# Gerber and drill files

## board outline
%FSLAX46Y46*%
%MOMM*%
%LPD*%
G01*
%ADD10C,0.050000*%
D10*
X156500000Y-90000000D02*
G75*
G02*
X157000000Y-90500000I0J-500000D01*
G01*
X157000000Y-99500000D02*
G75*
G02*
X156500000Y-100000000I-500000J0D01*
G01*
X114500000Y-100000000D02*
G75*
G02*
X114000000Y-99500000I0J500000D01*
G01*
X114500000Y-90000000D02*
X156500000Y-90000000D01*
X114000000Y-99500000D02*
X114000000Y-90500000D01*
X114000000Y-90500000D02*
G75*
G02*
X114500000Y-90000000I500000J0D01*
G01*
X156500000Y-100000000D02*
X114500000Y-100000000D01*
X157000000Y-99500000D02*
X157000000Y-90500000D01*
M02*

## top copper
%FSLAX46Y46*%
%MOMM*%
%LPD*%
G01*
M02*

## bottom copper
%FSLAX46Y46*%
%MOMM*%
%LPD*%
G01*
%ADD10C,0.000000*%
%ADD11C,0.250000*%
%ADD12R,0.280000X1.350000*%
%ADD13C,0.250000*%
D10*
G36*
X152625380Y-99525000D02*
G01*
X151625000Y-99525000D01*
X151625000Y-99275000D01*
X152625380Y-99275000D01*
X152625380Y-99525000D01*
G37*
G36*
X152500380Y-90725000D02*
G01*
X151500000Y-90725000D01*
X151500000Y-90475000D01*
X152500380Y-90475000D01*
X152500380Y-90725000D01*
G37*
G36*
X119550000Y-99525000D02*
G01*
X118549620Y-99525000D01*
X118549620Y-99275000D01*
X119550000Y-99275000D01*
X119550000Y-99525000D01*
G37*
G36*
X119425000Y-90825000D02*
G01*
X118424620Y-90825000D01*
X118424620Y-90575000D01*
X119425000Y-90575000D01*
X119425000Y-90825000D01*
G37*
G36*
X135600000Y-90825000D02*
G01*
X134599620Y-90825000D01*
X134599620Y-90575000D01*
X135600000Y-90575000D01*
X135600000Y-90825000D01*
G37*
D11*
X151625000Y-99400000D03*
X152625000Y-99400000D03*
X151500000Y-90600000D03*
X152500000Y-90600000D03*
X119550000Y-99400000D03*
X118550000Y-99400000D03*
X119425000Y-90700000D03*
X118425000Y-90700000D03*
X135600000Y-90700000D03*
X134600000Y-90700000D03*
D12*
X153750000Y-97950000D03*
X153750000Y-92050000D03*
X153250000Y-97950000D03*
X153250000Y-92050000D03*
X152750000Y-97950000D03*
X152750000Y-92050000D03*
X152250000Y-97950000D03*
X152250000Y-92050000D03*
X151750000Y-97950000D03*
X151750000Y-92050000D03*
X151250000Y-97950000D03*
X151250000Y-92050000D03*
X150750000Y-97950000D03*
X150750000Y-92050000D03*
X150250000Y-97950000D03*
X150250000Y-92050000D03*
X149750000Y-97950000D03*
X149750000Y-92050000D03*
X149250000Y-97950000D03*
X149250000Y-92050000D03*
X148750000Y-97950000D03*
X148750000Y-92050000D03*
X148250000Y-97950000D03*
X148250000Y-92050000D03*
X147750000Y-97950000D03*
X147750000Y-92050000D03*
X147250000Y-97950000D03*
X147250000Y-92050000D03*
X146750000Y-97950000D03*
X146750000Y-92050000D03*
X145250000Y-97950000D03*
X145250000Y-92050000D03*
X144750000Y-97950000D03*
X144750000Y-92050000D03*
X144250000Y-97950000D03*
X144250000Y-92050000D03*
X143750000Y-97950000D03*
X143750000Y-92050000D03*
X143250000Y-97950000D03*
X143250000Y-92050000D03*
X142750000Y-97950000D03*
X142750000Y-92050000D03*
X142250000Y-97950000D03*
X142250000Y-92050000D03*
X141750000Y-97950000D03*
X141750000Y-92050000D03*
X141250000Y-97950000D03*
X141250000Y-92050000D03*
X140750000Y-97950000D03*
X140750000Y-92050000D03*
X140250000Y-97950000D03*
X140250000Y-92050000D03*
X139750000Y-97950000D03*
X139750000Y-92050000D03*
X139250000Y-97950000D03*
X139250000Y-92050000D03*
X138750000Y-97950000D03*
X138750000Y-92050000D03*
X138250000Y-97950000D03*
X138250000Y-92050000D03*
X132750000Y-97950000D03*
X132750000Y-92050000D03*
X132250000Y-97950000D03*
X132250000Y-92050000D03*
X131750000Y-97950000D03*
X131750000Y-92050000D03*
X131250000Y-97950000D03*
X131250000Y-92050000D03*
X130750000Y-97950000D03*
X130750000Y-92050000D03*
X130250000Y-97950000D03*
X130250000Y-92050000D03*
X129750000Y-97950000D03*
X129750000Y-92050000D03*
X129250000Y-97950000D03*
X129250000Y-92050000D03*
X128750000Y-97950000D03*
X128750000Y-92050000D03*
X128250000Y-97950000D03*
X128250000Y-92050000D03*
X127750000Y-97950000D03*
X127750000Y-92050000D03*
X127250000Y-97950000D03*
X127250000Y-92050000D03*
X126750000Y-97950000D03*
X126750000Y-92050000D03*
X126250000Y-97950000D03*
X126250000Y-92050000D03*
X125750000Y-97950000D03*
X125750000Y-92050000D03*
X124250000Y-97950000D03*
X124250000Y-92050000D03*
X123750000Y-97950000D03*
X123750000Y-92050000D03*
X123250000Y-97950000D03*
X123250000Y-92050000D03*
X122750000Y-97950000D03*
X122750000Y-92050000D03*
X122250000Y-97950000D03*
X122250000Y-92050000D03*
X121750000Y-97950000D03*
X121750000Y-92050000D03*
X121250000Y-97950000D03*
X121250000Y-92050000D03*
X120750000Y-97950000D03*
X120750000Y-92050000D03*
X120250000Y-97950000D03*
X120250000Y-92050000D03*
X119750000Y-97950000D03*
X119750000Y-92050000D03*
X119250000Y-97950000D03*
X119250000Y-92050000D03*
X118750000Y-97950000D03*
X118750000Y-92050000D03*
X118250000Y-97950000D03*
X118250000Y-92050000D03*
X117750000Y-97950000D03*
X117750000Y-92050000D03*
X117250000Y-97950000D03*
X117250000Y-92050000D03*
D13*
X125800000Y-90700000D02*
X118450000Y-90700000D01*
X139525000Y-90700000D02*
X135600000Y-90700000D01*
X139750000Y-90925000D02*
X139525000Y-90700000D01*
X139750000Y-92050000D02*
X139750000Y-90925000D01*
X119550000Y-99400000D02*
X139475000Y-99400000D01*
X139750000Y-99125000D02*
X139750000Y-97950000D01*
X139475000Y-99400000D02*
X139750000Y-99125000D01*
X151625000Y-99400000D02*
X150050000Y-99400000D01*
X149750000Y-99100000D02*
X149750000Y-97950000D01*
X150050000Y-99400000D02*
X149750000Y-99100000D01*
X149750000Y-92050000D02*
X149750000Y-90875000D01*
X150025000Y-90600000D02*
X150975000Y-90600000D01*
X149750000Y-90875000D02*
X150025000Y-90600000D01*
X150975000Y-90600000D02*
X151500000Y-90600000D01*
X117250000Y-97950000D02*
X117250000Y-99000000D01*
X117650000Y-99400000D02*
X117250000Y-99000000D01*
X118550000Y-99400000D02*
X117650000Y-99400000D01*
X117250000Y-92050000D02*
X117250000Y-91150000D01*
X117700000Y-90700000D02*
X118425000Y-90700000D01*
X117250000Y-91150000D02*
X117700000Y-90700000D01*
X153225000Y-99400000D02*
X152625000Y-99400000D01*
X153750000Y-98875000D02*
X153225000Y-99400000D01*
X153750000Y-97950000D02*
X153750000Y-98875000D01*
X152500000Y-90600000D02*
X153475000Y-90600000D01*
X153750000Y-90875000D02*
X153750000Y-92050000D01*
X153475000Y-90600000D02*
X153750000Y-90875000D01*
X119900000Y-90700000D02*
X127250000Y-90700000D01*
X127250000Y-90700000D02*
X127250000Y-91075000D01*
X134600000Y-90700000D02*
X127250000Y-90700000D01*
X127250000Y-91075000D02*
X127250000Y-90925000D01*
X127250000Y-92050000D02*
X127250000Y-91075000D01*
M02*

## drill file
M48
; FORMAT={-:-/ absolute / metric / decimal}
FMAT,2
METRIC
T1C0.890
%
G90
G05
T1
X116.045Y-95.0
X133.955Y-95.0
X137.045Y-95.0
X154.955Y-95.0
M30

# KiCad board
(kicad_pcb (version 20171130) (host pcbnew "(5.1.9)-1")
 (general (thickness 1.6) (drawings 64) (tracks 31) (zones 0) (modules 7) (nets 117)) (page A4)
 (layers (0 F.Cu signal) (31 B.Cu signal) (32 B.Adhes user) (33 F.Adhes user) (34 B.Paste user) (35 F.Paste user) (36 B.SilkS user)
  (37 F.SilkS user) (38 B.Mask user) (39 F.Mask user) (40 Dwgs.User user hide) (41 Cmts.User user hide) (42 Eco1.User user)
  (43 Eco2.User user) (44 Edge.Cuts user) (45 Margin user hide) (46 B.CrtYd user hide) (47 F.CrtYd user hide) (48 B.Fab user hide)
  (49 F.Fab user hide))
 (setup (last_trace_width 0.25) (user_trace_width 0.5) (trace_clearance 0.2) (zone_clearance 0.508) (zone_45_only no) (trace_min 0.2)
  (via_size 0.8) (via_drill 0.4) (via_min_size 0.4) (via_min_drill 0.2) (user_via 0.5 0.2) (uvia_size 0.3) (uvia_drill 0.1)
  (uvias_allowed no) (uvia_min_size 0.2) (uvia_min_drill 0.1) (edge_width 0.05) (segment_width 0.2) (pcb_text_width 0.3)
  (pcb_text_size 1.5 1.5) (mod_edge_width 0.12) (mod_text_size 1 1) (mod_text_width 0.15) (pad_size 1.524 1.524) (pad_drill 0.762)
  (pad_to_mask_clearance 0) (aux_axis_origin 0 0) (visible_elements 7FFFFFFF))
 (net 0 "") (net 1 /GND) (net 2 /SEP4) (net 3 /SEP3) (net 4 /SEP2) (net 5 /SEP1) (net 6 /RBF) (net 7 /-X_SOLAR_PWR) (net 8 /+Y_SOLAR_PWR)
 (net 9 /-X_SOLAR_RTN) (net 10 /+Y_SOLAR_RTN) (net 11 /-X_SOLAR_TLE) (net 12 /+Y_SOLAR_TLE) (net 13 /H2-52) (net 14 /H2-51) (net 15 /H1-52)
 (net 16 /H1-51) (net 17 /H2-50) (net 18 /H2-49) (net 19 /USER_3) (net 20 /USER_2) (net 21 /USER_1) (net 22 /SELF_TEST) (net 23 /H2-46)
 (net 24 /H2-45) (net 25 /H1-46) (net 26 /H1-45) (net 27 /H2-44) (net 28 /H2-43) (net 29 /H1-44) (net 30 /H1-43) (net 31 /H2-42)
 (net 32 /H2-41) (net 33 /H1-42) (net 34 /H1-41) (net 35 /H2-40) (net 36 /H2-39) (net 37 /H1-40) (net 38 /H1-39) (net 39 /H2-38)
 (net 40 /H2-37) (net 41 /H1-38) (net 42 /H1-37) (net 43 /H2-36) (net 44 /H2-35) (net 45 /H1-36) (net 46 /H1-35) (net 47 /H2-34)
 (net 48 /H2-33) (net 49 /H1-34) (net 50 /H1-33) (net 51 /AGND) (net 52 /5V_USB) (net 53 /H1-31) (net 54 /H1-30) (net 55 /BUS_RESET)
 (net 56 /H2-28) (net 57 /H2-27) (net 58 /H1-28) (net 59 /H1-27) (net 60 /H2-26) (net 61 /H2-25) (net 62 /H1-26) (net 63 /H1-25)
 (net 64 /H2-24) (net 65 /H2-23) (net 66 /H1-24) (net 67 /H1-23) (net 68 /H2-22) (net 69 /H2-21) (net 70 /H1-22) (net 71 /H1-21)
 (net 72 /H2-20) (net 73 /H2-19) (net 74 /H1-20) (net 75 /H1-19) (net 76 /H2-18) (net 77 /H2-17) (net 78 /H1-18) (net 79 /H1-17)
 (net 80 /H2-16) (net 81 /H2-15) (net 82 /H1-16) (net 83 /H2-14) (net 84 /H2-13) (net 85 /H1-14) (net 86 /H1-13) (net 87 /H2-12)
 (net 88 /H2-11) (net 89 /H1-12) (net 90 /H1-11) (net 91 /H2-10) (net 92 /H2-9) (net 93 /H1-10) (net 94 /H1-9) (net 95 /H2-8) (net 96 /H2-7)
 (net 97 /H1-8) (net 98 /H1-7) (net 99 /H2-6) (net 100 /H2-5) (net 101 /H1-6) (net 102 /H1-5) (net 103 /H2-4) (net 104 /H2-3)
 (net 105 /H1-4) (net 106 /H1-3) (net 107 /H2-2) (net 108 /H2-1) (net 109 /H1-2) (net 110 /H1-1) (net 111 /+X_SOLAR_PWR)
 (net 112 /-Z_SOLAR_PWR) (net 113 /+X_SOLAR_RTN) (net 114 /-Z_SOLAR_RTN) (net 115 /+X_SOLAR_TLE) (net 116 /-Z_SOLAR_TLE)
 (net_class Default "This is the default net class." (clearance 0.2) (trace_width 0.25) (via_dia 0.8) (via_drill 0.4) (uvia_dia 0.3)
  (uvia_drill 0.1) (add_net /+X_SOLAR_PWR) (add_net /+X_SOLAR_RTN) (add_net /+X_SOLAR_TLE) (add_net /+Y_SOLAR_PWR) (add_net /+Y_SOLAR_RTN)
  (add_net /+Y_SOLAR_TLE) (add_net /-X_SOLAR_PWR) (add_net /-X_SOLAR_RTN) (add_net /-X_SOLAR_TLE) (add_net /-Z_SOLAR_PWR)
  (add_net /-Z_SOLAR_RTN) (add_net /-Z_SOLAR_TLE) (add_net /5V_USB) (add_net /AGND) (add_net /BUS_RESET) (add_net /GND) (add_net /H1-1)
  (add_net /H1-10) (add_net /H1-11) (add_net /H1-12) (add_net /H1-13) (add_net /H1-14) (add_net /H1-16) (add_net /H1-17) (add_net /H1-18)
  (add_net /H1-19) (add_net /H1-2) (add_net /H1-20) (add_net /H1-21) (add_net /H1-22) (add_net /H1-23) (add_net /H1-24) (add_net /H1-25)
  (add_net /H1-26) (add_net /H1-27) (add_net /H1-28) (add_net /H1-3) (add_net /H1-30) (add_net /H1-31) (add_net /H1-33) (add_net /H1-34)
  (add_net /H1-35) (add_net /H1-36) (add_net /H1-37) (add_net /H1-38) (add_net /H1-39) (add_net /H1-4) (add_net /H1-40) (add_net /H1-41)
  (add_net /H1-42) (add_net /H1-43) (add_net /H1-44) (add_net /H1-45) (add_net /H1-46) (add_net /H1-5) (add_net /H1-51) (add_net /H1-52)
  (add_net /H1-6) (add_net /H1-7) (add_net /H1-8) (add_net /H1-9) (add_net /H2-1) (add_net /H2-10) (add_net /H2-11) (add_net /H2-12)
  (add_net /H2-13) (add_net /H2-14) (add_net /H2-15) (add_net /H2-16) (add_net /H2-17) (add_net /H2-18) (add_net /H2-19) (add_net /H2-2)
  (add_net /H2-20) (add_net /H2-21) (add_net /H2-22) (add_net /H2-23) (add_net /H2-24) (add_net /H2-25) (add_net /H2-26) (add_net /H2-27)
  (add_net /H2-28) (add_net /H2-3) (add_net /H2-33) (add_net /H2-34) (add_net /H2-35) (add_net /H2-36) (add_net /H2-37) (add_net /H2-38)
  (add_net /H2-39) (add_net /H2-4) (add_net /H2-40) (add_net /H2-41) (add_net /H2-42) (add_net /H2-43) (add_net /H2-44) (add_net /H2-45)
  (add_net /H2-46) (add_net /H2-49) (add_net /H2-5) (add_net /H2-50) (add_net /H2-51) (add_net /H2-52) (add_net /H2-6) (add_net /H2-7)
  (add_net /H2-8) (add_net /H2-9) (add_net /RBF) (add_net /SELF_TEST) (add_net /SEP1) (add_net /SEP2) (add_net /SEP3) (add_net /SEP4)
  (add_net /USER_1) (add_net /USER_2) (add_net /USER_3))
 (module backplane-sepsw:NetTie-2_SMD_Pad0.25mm (layer B.Cu) (at 152.125 99.4 180)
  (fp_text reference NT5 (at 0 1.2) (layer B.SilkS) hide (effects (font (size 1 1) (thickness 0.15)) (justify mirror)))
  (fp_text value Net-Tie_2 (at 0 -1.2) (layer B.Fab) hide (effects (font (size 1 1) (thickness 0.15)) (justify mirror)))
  (fp_poly (pts (xy -0.50038 0.125) (xy 0.5 0.125) (xy 0.5 -0.125) (xy -0.50038 -0.125)) (layer B.Cu) (width 0))
  (pad 2 smd circle (at 0.5 0 180) (size 0.25 0.25) (layers B.Cu) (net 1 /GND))
  (pad 1 smd circle (at -0.5 0 180) (size 0.25 0.25) (layers B.Cu) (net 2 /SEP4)))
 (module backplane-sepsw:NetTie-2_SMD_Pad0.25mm (layer B.Cu) (at 152 90.6 180)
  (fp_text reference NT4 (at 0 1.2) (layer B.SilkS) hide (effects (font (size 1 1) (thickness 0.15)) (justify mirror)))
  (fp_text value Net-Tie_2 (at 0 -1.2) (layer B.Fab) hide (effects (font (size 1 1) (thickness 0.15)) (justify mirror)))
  (fp_poly (pts (xy -0.50038 0.125) (xy 0.5 0.125) (xy 0.5 -0.125) (xy -0.50038 -0.125)) (layer B.Cu) (width 0))
  (pad 2 smd circle (at 0.5 0 180) (size 0.25 0.25) (layers B.Cu) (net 1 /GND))
  (pad 1 smd circle (at -0.5 0 180) (size 0.25 0.25) (layers B.Cu) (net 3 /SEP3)))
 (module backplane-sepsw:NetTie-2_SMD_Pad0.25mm (layer B.Cu) (at 119.05 99.4)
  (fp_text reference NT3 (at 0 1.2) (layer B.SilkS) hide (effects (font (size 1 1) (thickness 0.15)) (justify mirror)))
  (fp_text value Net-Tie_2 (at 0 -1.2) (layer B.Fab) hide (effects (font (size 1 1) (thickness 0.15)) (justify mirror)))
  (fp_poly (pts (xy -0.50038 0.125) (xy 0.5 0.125) (xy 0.5 -0.125) (xy -0.50038 -0.125)) (layer B.Cu) (width 0))
  (pad 2 smd circle (at 0.5 0) (size 0.25 0.25) (layers B.Cu) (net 1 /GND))
  (pad 1 smd circle (at -0.5 0) (size 0.25 0.25) (layers B.Cu) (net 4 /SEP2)))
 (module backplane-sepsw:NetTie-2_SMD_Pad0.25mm (layer B.Cu) (at 118.925 90.7)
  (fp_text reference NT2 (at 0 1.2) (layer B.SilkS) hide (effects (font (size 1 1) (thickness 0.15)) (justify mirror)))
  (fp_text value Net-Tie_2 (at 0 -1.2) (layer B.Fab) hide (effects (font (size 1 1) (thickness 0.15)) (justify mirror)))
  (fp_poly (pts (xy -0.50038 0.125) (xy 0.5 0.125) (xy 0.5 -0.125) (xy -0.50038 -0.125)) (layer B.Cu) (width 0))
  (pad 2 smd circle (at 0.5 0) (size 0.25 0.25) (layers B.Cu) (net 1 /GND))
  (pad 1 smd circle (at -0.5 0) (size 0.25 0.25) (layers B.Cu) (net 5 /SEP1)))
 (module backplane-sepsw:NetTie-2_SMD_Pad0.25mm (layer B.Cu) (at 135.1 90.7)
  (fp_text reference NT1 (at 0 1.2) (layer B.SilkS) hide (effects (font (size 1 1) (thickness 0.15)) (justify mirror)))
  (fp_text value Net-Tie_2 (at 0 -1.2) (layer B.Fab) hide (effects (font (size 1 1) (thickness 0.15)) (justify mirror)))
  (fp_poly (pts (xy -0.50038 0.125) (xy 0.5 0.125) (xy 0.5 -0.125) (xy -0.50038 -0.125)) (layer B.Cu) (width 0))
  (pad 2 smd circle (at 0.5 0) (size 0.25 0.25) (layers B.Cu) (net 1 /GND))
  (pad 1 smd circle (at -0.5 0) (size 0.25 0.25) (layers B.Cu) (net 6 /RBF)))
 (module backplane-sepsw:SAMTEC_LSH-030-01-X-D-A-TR (layer B.Cu) (at 146 95)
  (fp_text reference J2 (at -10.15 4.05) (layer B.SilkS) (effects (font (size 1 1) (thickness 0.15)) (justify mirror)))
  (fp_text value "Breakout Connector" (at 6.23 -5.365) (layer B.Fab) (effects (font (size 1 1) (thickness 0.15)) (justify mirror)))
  (pad None np_thru_hole circle (at 8.955 0) (size 0.89 0.89) (drill 0.89) (layers *.Cu *.Mask))
  (pad None np_thru_hole circle (at -8.955 0) (size 0.89 0.89) (drill 0.89) (layers *.Cu *.Mask))
  (pad 60 smd rect (at 7.75 2.95) (size 0.28 1.35) (layers B.Cu B.Paste B.Mask) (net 2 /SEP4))
  (pad 59 smd rect (at 7.75 -2.95) (size 0.28 1.35) (layers B.Cu B.Paste B.Mask) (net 3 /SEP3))
  (pad 58 smd rect (at 7.25 2.95) (size 0.28 1.35) (layers B.Cu B.Paste B.Mask) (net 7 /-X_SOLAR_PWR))
  (pad 57 smd rect (at 7.25 -2.95) (size 0.28 1.35) (layers B.Cu B.Paste B.Mask) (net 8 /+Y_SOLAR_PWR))
  (pad 56 smd rect (at 6.75 2.95) (size 0.28 1.35) (layers B.Cu B.Paste B.Mask) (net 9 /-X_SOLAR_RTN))
  (pad 55 smd rect (at 6.75 -2.95) (size 0.28 1.35) (layers B.Cu B.Paste B.Mask) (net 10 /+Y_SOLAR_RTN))
  (pad 54 smd rect (at 6.25 2.95) (size 0.28 1.35) (layers B.Cu B.Paste B.Mask) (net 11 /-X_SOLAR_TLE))
  (pad 53 smd rect (at 6.25 -2.95) (size 0.28 1.35) (layers B.Cu B.Paste B.Mask) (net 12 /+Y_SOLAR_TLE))
  (pad 52 smd rect (at 5.75 2.95) (size 0.28 1.35) (layers B.Cu B.Paste B.Mask) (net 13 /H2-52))
  (pad 51 smd rect (at 5.75 -2.95) (size 0.28 1.35) (layers B.Cu B.Paste B.Mask) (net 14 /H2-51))
  (pad 50 smd rect (at 5.25 2.95) (size 0.28 1.35) (layers B.Cu B.Paste B.Mask) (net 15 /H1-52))
  (pad 49 smd rect (at 5.25 -2.95) (size 0.28 1.35) (layers B.Cu B.Paste B.Mask) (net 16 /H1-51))
  (pad 48 smd rect (at 4.75 2.95) (size 0.28 1.35) (layers B.Cu B.Paste B.Mask) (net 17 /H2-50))
  (pad 47 smd rect (at 4.75 -2.95) (size 0.28 1.35) (layers B.Cu B.Paste B.Mask) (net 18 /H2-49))
  (pad 46 smd rect (at 4.25 2.95) (size 0.28 1.35) (layers B.Cu B.Paste B.Mask) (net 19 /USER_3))
  (pad 45 smd rect (at 4.25 -2.95) (size 0.28 1.35) (layers B.Cu B.Paste B.Mask) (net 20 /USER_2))
  (pad 44 smd rect (at 3.75 2.95) (size 0.28 1.35) (layers B.Cu B.Paste B.Mask) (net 1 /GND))
  (pad 43 smd rect (at 3.75 -2.95) (size 0.28 1.35) (layers B.Cu B.Paste B.Mask) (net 1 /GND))
  (pad 42 smd rect (at 3.25 2.95) (size 0.28 1.35) (layers B.Cu B.Paste B.Mask) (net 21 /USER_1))
  (pad 41 smd rect (at 3.25 -2.95) (size 0.28 1.35) (layers B.Cu B.Paste B.Mask) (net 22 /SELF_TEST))
  (pad 40 smd rect (at 2.75 2.95) (size 0.28 1.35) (layers B.Cu B.Paste B.Mask) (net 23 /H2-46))
  (pad 39 smd rect (at 2.75 -2.95) (size 0.28 1.35) (layers B.Cu B.Paste B.Mask) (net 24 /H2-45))
  (pad 38 smd rect (at 2.25 2.95) (size 0.28 1.35) (layers B.Cu B.Paste B.Mask) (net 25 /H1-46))
  (pad 37 smd rect (at 2.25 -2.95) (size 0.28 1.35) (layers B.Cu B.Paste B.Mask) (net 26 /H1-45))
  (pad 36 smd rect (at 1.75 2.95) (size 0.28 1.35) (layers B.Cu B.Paste B.Mask) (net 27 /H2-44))
  (pad 35 smd rect (at 1.75 -2.95) (size 0.28 1.35) (layers B.Cu B.Paste B.Mask) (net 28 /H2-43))
  (pad 34 smd rect (at 1.25 2.95) (size 0.28 1.35) (layers B.Cu B.Paste B.Mask) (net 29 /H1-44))
  (pad 33 smd rect (at 1.25 -2.95) (size 0.28 1.35) (layers B.Cu B.Paste B.Mask) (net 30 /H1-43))
  (pad 32 smd rect (at 0.75 2.95) (size 0.28 1.35) (layers B.Cu B.Paste B.Mask) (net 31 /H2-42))
  (pad 31 smd rect (at 0.75 -2.95) (size 0.28 1.35) (layers B.Cu B.Paste B.Mask) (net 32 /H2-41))
  (pad 30 smd rect (at -0.75 2.95) (size 0.28 1.35) (layers B.Cu B.Paste B.Mask) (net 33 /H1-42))
  (pad 29 smd rect (at -0.75 -2.95) (size 0.28 1.35) (layers B.Cu B.Paste B.Mask) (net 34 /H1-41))
  (pad 28 smd rect (at -1.25 2.95) (size 0.28 1.35) (layers B.Cu B.Paste B.Mask) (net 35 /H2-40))
  (pad 27 smd rect (at -1.25 -2.95) (size 0.28 1.35) (layers B.Cu B.Paste B.Mask) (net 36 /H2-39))
  (pad 26 smd rect (at -1.75 2.95) (size 0.28 1.35) (layers B.Cu B.Paste B.Mask) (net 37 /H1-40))
  (pad 25 smd rect (at -1.75 -2.95) (size 0.28 1.35) (layers B.Cu B.Paste B.Mask) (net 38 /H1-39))
  (pad 24 smd rect (at -2.25 2.95) (size 0.28 1.35) (layers B.Cu B.Paste B.Mask) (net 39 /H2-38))
  (pad 23 smd rect (at -2.25 -2.95) (size 0.28 1.35) (layers B.Cu B.Paste B.Mask) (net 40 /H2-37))
  (pad 22 smd rect (at -2.75 2.95) (size 0.28 1.35) (layers B.Cu B.Paste B.Mask) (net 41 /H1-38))
  (pad 21 smd rect (at -2.75 -2.95) (size 0.28 1.35) (layers B.Cu B.Paste B.Mask) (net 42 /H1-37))
  (pad 20 smd rect (at -3.25 2.95) (size 0.28 1.35) (layers B.Cu B.Paste B.Mask) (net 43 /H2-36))
  (pad 19 smd rect (at -3.25 -2.95) (size 0.28 1.35) (layers B.Cu B.Paste B.Mask) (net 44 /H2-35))
  (pad 18 smd rect (at -3.75 2.95) (size 0.28 1.35) (layers B.Cu B.Paste B.Mask) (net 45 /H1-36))
  (pad 17 smd rect (at -3.75 -2.95) (size 0.28 1.35) (layers B.Cu B.Paste B.Mask) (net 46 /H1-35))
  (pad 16 smd rect (at -4.25 2.95) (size 0.28 1.35) (layers B.Cu B.Paste B.Mask) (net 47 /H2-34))
  (pad 15 smd rect (at -4.25 -2.95) (size 0.28 1.35) (layers B.Cu B.Paste B.Mask) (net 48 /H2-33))
  (pad 14 smd rect (at -4.75 2.95) (size 0.28 1.35) (layers B.Cu B.Paste B.Mask) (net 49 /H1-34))
  (pad 13 smd rect (at -4.75 -2.95) (size 0.28 1.35) (layers B.Cu B.Paste B.Mask) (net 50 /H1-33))
  (pad 12 smd rect (at -5.25 2.95) (size 0.28 1.35) (layers B.Cu B.Paste B.Mask) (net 1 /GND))
  (pad 11 smd rect (at -5.25 -2.95) (size 0.28 1.35) (layers B.Cu B.Paste B.Mask) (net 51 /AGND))
  (pad 10 smd rect (at -5.75 2.95) (size 0.28 1.35) (layers B.Cu B.Paste B.Mask) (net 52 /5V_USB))
  (pad 9 smd rect (at -5.75 -2.95) (size 0.28 1.35) (layers B.Cu B.Paste B.Mask) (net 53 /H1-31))
  (pad 8 smd rect (at -6.25 2.95) (size 0.28 1.35) (layers B.Cu B.Paste B.Mask) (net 1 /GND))
  (pad 7 smd rect (at -6.25 -2.95) (size 0.28 1.35) (layers B.Cu B.Paste B.Mask) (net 1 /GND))
  (pad 6 smd rect (at -6.75 2.95) (size 0.28 1.35) (layers B.Cu B.Paste B.Mask) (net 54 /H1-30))
  (pad 5 smd rect (at -6.75 -2.95) (size 0.28 1.35) (layers B.Cu B.Paste B.Mask) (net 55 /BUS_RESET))
  (pad 4 smd rect (at -7.25 2.95) (size 0.28 1.35) (layers B.Cu B.Paste B.Mask) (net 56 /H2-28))
  (pad 3 smd rect (at -7.25 -2.95) (size 0.28 1.35) (layers B.Cu B.Paste B.Mask) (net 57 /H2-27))
  (pad 2 smd rect (at -7.75 2.95) (size 0.28 1.35) (layers B.Cu B.Paste B.Mask) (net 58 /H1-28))
  (pad 1 smd rect (at -7.75 -2.95) (size 0.28 1.35) (layers B.Cu B.Paste B.Mask) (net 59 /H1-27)))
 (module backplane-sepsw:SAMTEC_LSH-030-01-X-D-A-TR (layer B.Cu) (at 125 95)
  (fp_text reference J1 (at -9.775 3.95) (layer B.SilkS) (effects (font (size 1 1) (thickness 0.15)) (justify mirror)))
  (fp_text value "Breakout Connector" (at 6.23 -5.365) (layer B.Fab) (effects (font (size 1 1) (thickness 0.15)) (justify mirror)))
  (pad None np_thru_hole circle (at 8.955 0) (size 0.89 0.89) (drill 0.89) (layers *.Cu *.Mask))
  (pad None np_thru_hole circle (at -8.955 0) (size 0.89 0.89) (drill 0.89) (layers *.Cu *.Mask))
  (pad 60 smd rect (at 7.75 2.95) (size 0.28 1.35) (layers B.Cu B.Paste B.Mask) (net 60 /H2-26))
  (pad 59 smd rect (at 7.75 -2.95) (size 0.28 1.35) (layers B.Cu B.Paste B.Mask) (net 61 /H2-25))
  (pad 58 smd rect (at 7.25 2.95) (size 0.28 1.35) (layers B.Cu B.Paste B.Mask) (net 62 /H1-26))
  (pad 57 smd rect (at 7.25 -2.95) (size 0.28 1.35) (layers B.Cu B.Paste B.Mask) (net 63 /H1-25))
  (pad 56 smd rect (at 6.75 2.95) (size 0.28 1.35) (layers B.Cu B.Paste B.Mask) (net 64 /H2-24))
  (pad 55 smd rect (at 6.75 -2.95) (size 0.28 1.35) (layers B.Cu B.Paste B.Mask) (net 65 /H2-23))
  (pad 54 smd rect (at 6.25 2.95) (size 0.28 1.35) (layers B.Cu B.Paste B.Mask) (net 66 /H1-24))
  (pad 53 smd rect (at 6.25 -2.95) (size 0.28 1.35) (layers B.Cu B.Paste B.Mask) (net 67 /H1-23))
  (pad 52 smd rect (at 5.75 2.95) (size 0.28 1.35) (layers B.Cu B.Paste B.Mask) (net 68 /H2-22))
  (pad 51 smd rect (at 5.75 -2.95) (size 0.28 1.35) (layers B.Cu B.Paste B.Mask) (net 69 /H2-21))
  (pad 50 smd rect (at 5.25 2.95) (size 0.28 1.35) (layers B.Cu B.Paste B.Mask) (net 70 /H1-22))
  (pad 49 smd rect (at 5.25 -2.95) (size 0.28 1.35) (layers B.Cu B.Paste B.Mask) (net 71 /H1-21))
  (pad 48 smd rect (at 4.75 2.95) (size 0.28 1.35) (layers B.Cu B.Paste B.Mask) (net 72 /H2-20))
  (pad 47 smd rect (at 4.75 -2.95) (size 0.28 1.35) (layers B.Cu B.Paste B.Mask) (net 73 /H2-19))
  (pad 46 smd rect (at 4.25 2.95) (size 0.28 1.35) (layers B.Cu B.Paste B.Mask) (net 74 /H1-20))
  (pad 45 smd rect (at 4.25 -2.95) (size 0.28 1.35) (layers B.Cu B.Paste B.Mask) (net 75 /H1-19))
  (pad 44 smd rect (at 3.75 2.95) (size 0.28 1.35) (layers B.Cu B.Paste B.Mask) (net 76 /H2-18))
  (pad 43 smd rect (at 3.75 -2.95) (size 0.28 1.35) (layers B.Cu B.Paste B.Mask) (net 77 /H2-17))
  (pad 42 smd rect (at 3.25 2.95) (size 0.28 1.35) (layers B.Cu B.Paste B.Mask) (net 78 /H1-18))
  (pad 41 smd rect (at 3.25 -2.95) (size 0.28 1.35) (layers B.Cu B.Paste B.Mask) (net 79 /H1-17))
  (pad 40 smd rect (at 2.75 2.95) (size 0.28 1.35) (layers B.Cu B.Paste B.Mask) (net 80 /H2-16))
  (pad 39 smd rect (at 2.75 -2.95) (size 0.28 1.35) (layers B.Cu B.Paste B.Mask) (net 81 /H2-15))
  (pad 38 smd rect (at 2.25 2.95) (size 0.28 1.35) (layers B.Cu B.Paste B.Mask) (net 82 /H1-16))
  (pad 37 smd rect (at 2.25 -2.95) (size 0.28 1.35) (layers B.Cu B.Paste B.Mask) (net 6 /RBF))
  (pad 36 smd rect (at 1.75 2.95) (size 0.28 1.35) (layers B.Cu B.Paste B.Mask) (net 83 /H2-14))
  (pad 35 smd rect (at 1.75 -2.95) (size 0.28 1.35) (layers B.Cu B.Paste B.Mask) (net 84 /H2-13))
  (pad 34 smd rect (at 1.25 2.95) (size 0.28 1.35) (layers B.Cu B.Paste B.Mask) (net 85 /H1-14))
  (pad 33 smd rect (at 1.25 -2.95) (size 0.28 1.35) (layers B.Cu B.Paste B.Mask) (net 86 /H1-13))
  (pad 32 smd rect (at 0.75 2.95) (size 0.28 1.35) (layers B.Cu B.Paste B.Mask) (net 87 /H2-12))
  (pad 31 smd rect (at 0.75 -2.95) (size 0.28 1.35) (layers B.Cu B.Paste B.Mask) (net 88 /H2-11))
  (pad 30 smd rect (at -0.75 2.95) (size 0.28 1.35) (layers B.Cu B.Paste B.Mask) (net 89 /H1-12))
  (pad 29 smd rect (at -0.75 -2.95) (size 0.28 1.35) (layers B.Cu B.Paste B.Mask) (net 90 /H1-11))
  (pad 28 smd rect (at -1.25 2.95) (size 0.28 1.35) (layers B.Cu B.Paste B.Mask) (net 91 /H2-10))
  (pad 27 smd rect (at -1.25 -2.95) (size 0.28 1.35) (layers B.Cu B.Paste B.Mask) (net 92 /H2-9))
  (pad 26 smd rect (at -1.75 2.95) (size 0.28 1.35) (layers B.Cu B.Paste B.Mask) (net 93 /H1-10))
  (pad 25 smd rect (at -1.75 -2.95) (size 0.28 1.35) (layers B.Cu B.Paste B.Mask) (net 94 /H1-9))
  (pad 24 smd rect (at -2.25 2.95) (size 0.28 1.35) (layers B.Cu B.Paste B.Mask) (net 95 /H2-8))
  (pad 23 smd rect (at -2.25 -2.95) (size 0.28 1.35) (layers B.Cu B.Paste B.Mask) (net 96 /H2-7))
  (pad 22 smd rect (at -2.75 2.95) (size 0.28 1.35) (layers B.Cu B.Paste B.Mask) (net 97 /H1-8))
  (pad 21 smd rect (at -2.75 -2.95) (size 0.28 1.35) (layers B.Cu B.Paste B.Mask) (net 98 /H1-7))
  (pad 20 smd rect (at -3.25 2.95) (size 0.28 1.35) (layers B.Cu B.Paste B.Mask) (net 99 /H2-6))
  (pad 19 smd rect (at -3.25 -2.95) (size 0.28 1.35) (layers B.Cu B.Paste B.Mask) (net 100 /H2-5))
  (pad 18 smd rect (at -3.75 2.95) (size 0.28 1.35) (layers B.Cu B.Paste B.Mask) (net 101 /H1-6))
  (pad 17 smd rect (at -3.75 -2.95) (size 0.28 1.35) (layers B.Cu B.Paste B.Mask) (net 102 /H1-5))
  (pad 16 smd rect (at -4.25 2.95) (size 0.28 1.35) (layers B.Cu B.Paste B.Mask) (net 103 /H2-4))
  (pad 15 smd rect (at -4.25 -2.95) (size 0.28 1.35) (layers B.Cu B.Paste B.Mask) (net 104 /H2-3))
  (pad 14 smd rect (at -4.75 2.95) (size 0.28 1.35) (layers B.Cu B.Paste B.Mask) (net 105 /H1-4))
  (pad 13 smd rect (at -4.75 -2.95) (size 0.28 1.35) (layers B.Cu B.Paste B.Mask) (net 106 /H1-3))
  (pad 12 smd rect (at -5.25 2.95) (size 0.28 1.35) (layers B.Cu B.Paste B.Mask) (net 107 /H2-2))
  (pad 11 smd rect (at -5.25 -2.95) (size 0.28 1.35) (layers B.Cu B.Paste B.Mask) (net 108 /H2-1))
  (pad 10 smd rect (at -5.75 2.95) (size 0.28 1.35) (layers B.Cu B.Paste B.Mask) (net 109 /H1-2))
  (pad 9 smd rect (at -5.75 -2.95) (size 0.28 1.35) (layers B.Cu B.Paste B.Mask) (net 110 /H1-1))
  (pad 8 smd rect (at -6.25 2.95) (size 0.28 1.35) (layers B.Cu B.Paste B.Mask) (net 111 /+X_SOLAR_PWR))
  (pad 7 smd rect (at -6.25 -2.95) (size 0.28 1.35) (layers B.Cu B.Paste B.Mask) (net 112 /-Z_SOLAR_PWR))
  (pad 6 smd rect (at -6.75 2.95) (size 0.28 1.35) (layers B.Cu B.Paste B.Mask) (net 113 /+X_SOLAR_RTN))
  (pad 5 smd rect (at -6.75 -2.95) (size 0.28 1.35) (layers B.Cu B.Paste B.Mask) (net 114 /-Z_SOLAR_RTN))
  (pad 4 smd rect (at -7.25 2.95) (size 0.28 1.35) (layers B.Cu B.Paste B.Mask) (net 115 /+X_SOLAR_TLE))
  (pad 3 smd rect (at -7.25 -2.95) (size 0.28 1.35) (layers B.Cu B.Paste B.Mask) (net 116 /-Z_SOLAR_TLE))
  (pad 2 smd rect (at -7.75 2.95) (size 0.28 1.35) (layers B.Cu B.Paste B.Mask) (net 4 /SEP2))
  (pad 1 smd rect (at -7.75 -2.95) (size 0.28 1.35) (layers B.Cu B.Paste B.Mask) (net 5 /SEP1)))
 (gr_arc (start 156.5 90.5) (end 157 90.5) (angle -90) (layer Edge.Cuts) (width 0.05))
 (gr_arc (start 156.5 99.5) (end 156.5 100) (angle -90) (layer Edge.Cuts) (width 0.05))
 (gr_arc (start 114.5 99.5) (end 114.5 100) (angle 90) (layer Edge.Cuts) (width 0.05))
 (gr_line (start 114.5 90) (end 156.5 90) (layer Edge.Cuts) (width 0.05))
 (gr_line (start 114 99.5) (end 114 90.5) (layer Edge.Cuts) (width 0.05))
 (gr_arc (start 114.5 90.5) (end 114.5 90) (angle -90) (layer Edge.Cuts) (width 0.05))
 (gr_line (start 156.5 100) (end 114.5 100) (layer Edge.Cuts) (width 0.05))
 (gr_line (start 157 99.5) (end 157 90.5) (layer Edge.Cuts) (width 0.05))
 (segment (start 125.8 90.7) (end 118.45 90.7) (width 0.25) (layer B.Cu) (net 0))
 (segment (start 139.525 90.7) (end 135.6 90.7) (width 0.25) (layer B.Cu) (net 1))
 (segment (start 139.75 90.925) (end 139.525 90.7) (width 0.25) (layer B.Cu) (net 1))
 (segment (start 139.75 92.05) (end 139.75 90.925) (width 0.25) (layer B.Cu) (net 1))
 (segment (start 119.55 99.4) (end 139.475 99.4) (width 0.25) (layer B.Cu) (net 1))
 (segment (start 139.75 99.125) (end 139.75 97.95) (width 0.25) (layer B.Cu) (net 1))
 (segment (start 139.475 99.4) (end 139.75 99.125) (width 0.25) (layer B.Cu) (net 1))
 (segment (start 151.625 99.4) (end 150.05 99.4) (width 0.25) (layer B.Cu) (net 1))
 (segment (start 149.75 99.1) (end 149.75 97.95) (width 0.25) (layer B.Cu) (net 1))
 (segment (start 150.05 99.4) (end 149.75 99.1) (width 0.25) (layer B.Cu) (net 1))
 (segment (start 149.75 92.05) (end 149.75 90.875) (width 0.25) (layer B.Cu) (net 1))
 (segment (start 150.025 90.6) (end 150.975 90.6) (width 0.25) (layer B.Cu) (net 1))
 (segment (start 149.75 90.875) (end 150.025 90.6) (width 0.25) (layer B.Cu) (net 1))
 (segment (start 150.975 90.6) (end 151.5 90.6) (width 0.25) (layer B.Cu) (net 1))
 (segment (start 117.25 97.95) (end 117.25 99) (width 0.25) (layer B.Cu) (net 4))
 (segment (start 117.65 99.4) (end 117.25 99) (width 0.25) (layer B.Cu) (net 4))
 (segment (start 118.55 99.4) (end 117.65 99.4) (width 0.25) (layer B.Cu) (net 4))
 (segment (start 117.25 92.05) (end 117.25 91.15) (width 0.25) (layer B.Cu) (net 5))
 (segment (start 117.7 90.7) (end 118.425 90.7) (width 0.25) (layer B.Cu) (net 5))
 (segment (start 117.25 91.15) (end 117.7 90.7) (width 0.25) (layer B.Cu) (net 5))
 (segment (start 153.225 99.4) (end 152.625 99.4) (width 0.25) (layer B.Cu) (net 2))
 (segment (start 153.75 98.875) (end 153.225 99.4) (width 0.25) (layer B.Cu) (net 2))
 (segment (start 153.75 97.95) (end 153.75 98.875) (width 0.25) (layer B.Cu) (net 2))
 (segment (start 152.5 90.6) (end 153.475 90.6) (width 0.25) (layer B.Cu) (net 3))
 (segment (start 153.75 90.875) (end 153.75 92.05) (width 0.25) (layer B.Cu) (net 3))
 (segment (start 153.475 90.6) (end 153.75 90.875) (width 0.25) (layer B.Cu) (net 3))
 (segment (start 119.9 90.7) (end 127.25 90.7) (width 0.25) (layer B.Cu) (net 6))
 (segment (start 127.25 90.7) (end 127.25 91.075) (width 0.25) (layer B.Cu) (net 6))
 (segment (start 134.6 90.7) (end 127.25 90.7) (width 0.25) (layer B.Cu) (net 6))
 (segment (start 127.25 91.075) (end 127.25 90.925) (width 0.25) (layer B.Cu) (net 6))
 (segment (start 127.25 92.05) (end 127.25 91.075) (width 0.25) (layer B.Cu) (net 6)))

